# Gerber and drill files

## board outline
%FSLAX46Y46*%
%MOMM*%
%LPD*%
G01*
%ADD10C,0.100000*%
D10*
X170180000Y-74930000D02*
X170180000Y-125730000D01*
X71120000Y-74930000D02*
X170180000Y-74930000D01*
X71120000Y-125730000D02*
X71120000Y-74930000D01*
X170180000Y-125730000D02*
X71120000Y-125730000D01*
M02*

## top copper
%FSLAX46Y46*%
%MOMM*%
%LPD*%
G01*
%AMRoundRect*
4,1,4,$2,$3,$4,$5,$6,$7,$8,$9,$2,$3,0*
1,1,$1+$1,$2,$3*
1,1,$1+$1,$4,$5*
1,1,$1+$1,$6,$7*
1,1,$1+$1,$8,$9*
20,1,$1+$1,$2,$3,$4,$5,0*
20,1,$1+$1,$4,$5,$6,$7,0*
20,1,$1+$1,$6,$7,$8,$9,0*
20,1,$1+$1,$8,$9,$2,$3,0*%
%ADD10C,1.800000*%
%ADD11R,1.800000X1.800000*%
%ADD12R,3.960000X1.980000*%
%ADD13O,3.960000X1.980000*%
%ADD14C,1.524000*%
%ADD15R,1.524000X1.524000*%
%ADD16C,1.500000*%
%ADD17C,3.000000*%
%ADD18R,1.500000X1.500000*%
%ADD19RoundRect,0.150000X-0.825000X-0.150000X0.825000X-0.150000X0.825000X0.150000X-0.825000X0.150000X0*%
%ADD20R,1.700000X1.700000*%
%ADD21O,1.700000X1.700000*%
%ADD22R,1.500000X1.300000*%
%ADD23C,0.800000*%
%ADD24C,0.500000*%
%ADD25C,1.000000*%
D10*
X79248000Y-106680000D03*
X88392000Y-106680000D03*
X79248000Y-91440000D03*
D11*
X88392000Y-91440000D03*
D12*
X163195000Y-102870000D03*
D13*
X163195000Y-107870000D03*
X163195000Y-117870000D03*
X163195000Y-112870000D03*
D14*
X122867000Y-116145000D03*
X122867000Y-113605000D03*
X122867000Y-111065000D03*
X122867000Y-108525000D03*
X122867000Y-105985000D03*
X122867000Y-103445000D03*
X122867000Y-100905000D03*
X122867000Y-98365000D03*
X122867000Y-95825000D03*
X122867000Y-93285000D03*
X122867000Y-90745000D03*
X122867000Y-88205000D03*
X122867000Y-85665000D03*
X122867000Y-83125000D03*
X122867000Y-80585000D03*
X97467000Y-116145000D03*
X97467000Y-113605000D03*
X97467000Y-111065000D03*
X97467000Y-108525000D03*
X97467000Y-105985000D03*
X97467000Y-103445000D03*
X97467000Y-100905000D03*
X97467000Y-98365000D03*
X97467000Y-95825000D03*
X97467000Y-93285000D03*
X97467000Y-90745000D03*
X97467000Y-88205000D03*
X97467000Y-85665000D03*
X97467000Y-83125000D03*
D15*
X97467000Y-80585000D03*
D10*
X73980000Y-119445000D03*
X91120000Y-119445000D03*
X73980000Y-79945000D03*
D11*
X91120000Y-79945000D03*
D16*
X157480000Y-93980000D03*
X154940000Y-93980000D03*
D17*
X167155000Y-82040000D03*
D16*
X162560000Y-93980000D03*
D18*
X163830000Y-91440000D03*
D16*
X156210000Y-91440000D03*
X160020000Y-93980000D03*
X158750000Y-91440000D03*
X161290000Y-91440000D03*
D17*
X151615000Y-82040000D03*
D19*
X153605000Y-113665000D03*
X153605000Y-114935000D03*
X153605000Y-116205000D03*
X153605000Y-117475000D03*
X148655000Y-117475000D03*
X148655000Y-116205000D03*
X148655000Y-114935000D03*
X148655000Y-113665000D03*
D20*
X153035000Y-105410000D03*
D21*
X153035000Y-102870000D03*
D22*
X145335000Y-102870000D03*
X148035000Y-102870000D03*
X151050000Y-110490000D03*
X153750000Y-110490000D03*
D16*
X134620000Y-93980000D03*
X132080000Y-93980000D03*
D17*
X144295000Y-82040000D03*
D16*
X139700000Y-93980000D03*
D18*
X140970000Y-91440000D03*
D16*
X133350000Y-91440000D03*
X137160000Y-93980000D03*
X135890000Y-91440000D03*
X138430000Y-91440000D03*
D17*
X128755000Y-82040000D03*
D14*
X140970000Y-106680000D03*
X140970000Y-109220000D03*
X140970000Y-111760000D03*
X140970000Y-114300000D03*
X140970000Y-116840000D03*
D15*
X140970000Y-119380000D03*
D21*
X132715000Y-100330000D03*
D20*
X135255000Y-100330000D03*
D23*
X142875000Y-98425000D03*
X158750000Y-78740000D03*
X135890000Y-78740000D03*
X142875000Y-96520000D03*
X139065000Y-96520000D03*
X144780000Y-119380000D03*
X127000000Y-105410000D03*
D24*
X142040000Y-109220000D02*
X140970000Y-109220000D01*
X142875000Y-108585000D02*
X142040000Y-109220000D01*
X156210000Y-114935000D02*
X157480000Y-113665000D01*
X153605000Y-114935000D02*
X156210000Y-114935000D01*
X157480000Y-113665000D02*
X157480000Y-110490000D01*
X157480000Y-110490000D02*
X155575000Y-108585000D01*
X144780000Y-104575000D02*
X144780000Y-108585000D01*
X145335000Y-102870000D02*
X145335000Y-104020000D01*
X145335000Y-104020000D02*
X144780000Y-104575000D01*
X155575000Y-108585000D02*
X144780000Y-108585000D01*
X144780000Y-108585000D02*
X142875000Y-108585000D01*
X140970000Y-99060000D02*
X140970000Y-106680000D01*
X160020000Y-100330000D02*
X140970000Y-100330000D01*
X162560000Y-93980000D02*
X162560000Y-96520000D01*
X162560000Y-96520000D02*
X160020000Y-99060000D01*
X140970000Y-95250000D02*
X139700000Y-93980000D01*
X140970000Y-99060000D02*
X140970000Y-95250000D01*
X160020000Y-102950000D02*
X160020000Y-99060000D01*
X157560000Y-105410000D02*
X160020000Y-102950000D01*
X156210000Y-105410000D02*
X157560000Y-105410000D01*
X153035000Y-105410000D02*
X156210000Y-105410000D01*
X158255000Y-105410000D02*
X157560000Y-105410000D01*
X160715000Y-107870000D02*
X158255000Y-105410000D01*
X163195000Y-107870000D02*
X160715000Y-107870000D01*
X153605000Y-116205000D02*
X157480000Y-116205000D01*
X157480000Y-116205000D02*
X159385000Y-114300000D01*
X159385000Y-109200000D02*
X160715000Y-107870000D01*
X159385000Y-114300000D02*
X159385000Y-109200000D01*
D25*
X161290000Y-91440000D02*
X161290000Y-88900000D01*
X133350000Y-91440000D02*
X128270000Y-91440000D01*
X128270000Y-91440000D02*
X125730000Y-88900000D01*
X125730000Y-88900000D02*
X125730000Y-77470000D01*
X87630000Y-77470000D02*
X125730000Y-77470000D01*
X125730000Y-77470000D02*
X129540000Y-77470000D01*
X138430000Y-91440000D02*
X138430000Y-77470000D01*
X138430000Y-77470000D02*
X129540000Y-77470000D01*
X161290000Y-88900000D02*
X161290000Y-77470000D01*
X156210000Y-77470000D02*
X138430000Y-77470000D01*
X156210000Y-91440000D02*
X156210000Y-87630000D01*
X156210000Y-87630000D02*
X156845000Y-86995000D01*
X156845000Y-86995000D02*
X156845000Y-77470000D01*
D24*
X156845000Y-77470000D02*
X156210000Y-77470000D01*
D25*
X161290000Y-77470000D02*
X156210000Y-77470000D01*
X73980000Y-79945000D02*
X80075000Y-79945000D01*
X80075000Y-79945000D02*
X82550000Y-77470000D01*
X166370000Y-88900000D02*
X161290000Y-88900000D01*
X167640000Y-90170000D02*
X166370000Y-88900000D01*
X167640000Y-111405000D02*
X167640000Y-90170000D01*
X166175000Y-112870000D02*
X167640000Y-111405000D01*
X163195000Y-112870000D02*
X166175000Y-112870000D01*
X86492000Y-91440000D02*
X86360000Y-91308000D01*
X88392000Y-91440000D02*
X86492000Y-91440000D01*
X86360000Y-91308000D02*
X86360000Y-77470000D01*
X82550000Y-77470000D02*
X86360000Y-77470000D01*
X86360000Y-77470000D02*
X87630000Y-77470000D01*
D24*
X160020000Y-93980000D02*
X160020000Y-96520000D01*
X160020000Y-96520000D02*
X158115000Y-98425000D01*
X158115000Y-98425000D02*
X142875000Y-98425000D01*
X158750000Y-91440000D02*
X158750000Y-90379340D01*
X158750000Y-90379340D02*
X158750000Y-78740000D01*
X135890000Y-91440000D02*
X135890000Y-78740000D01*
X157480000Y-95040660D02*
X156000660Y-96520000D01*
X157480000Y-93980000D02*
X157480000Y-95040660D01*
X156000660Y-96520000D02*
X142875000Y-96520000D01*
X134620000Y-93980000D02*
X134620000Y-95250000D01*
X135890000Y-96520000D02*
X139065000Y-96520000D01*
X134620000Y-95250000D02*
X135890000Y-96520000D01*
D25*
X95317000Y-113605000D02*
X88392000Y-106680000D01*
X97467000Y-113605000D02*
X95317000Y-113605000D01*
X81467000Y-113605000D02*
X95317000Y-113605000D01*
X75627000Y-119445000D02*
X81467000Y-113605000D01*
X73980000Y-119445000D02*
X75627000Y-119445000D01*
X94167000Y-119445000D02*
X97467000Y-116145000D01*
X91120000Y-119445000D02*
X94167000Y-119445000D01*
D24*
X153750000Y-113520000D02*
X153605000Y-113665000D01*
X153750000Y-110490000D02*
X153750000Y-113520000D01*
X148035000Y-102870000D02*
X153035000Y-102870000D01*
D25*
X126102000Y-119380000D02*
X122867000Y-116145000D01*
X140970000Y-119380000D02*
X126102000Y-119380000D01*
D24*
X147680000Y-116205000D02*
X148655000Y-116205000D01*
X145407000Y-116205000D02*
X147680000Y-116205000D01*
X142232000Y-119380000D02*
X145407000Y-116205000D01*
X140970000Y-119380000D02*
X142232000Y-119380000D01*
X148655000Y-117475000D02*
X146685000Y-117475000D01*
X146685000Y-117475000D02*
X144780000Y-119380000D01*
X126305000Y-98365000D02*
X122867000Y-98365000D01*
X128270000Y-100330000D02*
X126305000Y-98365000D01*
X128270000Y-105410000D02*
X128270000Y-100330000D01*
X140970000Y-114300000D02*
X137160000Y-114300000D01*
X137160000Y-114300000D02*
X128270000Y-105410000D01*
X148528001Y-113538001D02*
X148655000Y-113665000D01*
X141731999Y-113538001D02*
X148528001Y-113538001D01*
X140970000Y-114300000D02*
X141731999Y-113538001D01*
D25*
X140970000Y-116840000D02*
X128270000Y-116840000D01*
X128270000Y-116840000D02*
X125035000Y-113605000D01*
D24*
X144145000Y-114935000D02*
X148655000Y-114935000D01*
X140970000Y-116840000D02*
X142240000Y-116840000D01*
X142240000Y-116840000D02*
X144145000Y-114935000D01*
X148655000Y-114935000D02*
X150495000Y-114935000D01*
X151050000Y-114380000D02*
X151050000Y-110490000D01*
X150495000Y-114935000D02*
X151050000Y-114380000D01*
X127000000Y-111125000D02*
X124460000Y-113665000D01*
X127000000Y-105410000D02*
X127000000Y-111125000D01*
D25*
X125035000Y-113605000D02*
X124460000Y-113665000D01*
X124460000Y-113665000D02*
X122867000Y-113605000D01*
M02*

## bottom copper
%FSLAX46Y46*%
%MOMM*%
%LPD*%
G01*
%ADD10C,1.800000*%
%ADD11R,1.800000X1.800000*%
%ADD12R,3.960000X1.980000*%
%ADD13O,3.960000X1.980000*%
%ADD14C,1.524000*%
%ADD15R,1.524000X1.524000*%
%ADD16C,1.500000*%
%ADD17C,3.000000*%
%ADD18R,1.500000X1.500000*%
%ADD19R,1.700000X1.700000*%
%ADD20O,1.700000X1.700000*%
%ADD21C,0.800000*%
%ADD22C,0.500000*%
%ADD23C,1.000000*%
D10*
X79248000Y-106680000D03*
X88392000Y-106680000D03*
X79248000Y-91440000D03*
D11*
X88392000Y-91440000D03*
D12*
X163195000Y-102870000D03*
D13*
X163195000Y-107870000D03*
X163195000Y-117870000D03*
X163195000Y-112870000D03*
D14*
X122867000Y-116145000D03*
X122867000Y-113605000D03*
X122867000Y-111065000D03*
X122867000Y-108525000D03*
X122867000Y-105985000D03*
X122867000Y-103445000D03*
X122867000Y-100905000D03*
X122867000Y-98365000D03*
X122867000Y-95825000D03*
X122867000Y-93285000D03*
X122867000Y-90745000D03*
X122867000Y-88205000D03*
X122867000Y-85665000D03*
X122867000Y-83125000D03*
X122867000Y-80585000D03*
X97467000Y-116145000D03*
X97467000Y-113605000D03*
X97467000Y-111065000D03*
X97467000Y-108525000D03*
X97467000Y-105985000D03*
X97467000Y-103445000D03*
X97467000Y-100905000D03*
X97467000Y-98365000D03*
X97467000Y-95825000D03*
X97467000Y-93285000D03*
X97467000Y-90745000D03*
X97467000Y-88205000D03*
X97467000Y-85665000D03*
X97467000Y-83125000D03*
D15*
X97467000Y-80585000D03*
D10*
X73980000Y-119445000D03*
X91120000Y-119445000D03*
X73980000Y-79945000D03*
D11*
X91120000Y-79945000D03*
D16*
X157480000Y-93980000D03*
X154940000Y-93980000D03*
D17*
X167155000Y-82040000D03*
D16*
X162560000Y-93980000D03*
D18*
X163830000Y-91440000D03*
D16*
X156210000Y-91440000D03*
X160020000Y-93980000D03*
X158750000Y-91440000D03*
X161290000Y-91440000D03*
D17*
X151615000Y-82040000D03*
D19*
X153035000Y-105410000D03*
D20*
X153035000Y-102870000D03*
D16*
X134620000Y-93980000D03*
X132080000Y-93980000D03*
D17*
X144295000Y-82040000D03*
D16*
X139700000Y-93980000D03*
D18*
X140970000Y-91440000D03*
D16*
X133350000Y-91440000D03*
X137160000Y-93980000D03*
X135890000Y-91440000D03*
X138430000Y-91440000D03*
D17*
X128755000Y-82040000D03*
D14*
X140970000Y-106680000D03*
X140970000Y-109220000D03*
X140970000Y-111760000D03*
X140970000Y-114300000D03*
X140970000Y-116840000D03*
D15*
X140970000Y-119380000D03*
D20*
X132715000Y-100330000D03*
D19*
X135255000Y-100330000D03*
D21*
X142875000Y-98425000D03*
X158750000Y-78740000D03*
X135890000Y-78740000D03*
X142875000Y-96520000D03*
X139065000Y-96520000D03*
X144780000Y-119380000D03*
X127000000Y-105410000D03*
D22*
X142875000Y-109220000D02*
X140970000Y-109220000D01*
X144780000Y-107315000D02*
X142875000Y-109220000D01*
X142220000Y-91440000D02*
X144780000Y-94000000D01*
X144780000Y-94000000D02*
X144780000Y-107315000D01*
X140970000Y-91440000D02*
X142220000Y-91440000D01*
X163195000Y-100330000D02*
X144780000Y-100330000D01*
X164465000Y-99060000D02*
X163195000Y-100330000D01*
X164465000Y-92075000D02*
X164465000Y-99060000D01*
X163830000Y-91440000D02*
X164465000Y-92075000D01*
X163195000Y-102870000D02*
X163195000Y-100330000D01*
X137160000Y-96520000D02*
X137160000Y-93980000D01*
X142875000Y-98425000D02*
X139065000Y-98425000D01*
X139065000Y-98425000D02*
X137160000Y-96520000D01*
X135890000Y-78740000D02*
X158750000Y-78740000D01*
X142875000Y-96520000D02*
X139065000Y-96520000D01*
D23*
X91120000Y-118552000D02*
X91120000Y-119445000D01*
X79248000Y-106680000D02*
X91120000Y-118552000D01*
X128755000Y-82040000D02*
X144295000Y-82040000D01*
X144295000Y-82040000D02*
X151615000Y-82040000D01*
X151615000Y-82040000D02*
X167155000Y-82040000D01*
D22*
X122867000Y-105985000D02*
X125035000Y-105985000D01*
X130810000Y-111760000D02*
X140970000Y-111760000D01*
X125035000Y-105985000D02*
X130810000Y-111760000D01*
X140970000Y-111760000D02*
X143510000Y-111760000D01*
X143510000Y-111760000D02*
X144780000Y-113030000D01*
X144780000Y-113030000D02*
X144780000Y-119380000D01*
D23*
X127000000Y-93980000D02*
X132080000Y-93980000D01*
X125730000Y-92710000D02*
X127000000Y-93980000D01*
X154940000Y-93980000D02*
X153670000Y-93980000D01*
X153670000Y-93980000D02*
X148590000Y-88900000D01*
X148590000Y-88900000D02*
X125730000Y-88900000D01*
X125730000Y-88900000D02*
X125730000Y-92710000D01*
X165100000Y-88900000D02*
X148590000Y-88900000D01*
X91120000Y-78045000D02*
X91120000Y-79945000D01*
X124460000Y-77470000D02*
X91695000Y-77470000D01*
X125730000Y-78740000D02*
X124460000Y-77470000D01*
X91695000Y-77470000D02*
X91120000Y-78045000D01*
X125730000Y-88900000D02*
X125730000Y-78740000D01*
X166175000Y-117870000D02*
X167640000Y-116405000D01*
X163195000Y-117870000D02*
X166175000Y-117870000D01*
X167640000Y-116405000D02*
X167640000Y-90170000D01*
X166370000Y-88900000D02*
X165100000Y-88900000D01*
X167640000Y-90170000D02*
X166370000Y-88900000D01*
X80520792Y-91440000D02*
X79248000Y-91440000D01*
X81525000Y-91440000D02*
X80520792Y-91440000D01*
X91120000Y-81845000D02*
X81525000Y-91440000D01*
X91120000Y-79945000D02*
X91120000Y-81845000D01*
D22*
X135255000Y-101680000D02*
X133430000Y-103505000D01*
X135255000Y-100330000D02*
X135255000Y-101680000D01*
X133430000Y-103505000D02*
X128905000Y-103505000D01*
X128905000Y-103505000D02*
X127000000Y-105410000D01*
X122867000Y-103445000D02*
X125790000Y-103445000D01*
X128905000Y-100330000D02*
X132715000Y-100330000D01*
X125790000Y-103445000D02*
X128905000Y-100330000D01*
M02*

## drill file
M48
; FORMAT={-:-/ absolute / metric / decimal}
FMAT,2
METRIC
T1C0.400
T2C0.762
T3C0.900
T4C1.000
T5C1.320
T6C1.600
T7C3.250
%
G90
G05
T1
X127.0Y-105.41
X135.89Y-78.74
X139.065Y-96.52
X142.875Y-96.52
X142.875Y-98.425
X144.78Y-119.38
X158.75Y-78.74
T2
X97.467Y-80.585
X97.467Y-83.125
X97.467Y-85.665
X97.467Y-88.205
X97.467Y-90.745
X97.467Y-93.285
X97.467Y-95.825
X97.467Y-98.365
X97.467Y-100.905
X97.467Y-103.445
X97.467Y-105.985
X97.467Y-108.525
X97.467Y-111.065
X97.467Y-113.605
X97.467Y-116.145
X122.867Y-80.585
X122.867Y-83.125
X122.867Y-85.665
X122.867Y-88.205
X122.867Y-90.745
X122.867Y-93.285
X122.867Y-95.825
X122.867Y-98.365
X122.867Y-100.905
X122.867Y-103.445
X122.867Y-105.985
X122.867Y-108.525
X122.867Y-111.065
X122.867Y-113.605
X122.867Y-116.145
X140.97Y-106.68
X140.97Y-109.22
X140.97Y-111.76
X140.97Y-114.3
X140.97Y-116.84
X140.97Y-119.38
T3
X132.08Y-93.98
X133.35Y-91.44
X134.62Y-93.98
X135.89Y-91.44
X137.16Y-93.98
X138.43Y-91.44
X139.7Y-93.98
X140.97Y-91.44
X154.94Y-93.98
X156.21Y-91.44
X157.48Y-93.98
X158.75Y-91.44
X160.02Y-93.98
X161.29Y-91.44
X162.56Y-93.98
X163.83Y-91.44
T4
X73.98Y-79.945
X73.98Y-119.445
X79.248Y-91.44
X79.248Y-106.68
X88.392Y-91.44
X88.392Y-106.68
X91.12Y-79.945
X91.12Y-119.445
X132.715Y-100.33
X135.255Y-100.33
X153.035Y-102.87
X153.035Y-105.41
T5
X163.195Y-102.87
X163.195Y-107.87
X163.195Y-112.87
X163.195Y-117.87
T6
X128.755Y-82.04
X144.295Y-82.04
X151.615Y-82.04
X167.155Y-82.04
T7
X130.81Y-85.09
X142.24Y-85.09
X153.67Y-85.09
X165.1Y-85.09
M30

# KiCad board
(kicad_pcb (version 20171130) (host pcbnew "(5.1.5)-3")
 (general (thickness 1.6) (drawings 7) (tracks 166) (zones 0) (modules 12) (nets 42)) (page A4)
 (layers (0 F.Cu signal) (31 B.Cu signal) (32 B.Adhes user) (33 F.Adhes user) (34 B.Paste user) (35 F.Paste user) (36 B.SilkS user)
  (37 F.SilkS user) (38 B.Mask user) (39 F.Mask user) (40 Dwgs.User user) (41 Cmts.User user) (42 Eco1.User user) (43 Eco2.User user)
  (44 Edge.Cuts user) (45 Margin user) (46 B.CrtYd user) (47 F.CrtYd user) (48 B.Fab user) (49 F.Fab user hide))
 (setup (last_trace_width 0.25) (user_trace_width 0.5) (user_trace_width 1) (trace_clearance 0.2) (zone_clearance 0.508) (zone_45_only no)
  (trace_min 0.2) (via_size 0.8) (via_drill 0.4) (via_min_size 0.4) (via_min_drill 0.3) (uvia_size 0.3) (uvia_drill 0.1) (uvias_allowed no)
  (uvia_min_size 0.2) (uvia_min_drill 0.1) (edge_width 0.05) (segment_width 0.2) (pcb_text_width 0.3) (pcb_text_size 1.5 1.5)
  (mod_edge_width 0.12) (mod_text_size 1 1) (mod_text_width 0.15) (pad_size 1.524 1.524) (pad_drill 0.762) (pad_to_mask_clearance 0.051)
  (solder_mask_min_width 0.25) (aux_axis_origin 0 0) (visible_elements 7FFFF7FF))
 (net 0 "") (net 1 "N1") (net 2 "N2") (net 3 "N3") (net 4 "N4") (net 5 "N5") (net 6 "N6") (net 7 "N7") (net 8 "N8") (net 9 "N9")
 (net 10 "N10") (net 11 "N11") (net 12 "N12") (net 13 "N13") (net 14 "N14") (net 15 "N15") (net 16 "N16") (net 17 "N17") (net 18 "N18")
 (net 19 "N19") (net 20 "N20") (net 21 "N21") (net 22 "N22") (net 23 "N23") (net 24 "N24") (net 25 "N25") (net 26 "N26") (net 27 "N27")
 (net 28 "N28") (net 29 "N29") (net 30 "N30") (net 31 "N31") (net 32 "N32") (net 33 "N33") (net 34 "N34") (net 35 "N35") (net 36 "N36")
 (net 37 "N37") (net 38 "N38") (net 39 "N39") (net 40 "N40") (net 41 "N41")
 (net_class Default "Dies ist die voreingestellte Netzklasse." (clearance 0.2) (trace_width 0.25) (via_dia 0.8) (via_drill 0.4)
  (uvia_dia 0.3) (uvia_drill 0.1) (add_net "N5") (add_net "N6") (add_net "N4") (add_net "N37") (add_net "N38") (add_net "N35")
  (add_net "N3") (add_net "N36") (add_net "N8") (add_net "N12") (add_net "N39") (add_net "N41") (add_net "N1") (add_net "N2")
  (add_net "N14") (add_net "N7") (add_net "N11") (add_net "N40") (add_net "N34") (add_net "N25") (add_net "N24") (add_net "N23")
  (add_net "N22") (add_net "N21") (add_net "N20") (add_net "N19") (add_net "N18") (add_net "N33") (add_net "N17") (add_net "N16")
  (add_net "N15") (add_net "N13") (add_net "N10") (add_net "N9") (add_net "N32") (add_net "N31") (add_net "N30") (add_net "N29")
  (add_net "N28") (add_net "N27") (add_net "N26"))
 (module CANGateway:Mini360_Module (layer F.Cu) (at 83.82 99.06 270)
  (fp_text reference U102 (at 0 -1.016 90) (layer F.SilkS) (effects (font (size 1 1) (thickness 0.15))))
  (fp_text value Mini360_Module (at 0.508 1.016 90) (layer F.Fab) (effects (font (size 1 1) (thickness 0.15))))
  (pad 4 thru_hole circle (at 7.62 4.572 270) (size 1.8 1.8) (drill 1) (layers *.Cu *.Mask) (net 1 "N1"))
  (pad 3 thru_hole circle (at 7.62 -4.572 270) (size 1.8 1.8) (drill 1) (layers *.Cu *.Mask) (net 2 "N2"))
  (pad 2 thru_hole circle (at -7.62 4.572 270) (size 1.8 1.8) (drill 1) (layers *.Cu *.Mask) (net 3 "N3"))
  (pad 1 thru_hole rect (at -7.62 -4.572 270) (size 1.8 1.8) (drill 1) (layers *.Cu *.Mask) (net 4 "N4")))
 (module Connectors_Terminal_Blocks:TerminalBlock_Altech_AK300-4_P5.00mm (layer F.Cu) (at 163.195 102.87 270)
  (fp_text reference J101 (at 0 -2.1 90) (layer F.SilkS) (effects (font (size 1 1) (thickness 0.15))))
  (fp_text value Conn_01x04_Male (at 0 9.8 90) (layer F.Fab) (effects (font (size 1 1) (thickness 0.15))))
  (pad 1 thru_hole rect (at 0 0 270) (size 1.98 3.96) (drill 1.32) (layers *.Cu *.Mask) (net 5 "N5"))
  (pad 2 thru_hole oval (at 5 0 270) (size 1.98 3.96) (drill 1.32) (layers *.Cu *.Mask) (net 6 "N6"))
  (pad 4 thru_hole oval (at 15 0 270) (size 1.98 3.96) (drill 1.32) (layers *.Cu *.Mask) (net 3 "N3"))
  (pad 3 thru_hole oval (at 10 0 270) (size 1.98 3.96) (drill 1.32) (layers *.Cu *.Mask) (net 4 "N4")))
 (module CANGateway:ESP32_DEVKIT (layer F.Cu) (at 110.167 95.825)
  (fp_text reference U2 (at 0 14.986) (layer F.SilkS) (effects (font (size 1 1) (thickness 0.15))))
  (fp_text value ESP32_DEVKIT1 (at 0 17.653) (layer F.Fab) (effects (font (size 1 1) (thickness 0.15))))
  (pad 30 thru_hole circle (at 12.7 20.32) (size 1.524 1.524) (drill 0.762) (layers *.Cu *.Mask) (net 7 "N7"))
  (pad 29 thru_hole circle (at 12.7 17.78) (size 1.524 1.524) (drill 0.762) (layers *.Cu *.Mask) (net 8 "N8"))
  (pad 28 thru_hole circle (at 12.7 15.24) (size 1.524 1.524) (drill 0.762) (layers *.Cu *.Mask) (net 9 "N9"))
  (pad 27 thru_hole circle (at 12.7 12.7) (size 1.524 1.524) (drill 0.762) (layers *.Cu *.Mask) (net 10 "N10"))
  (pad 26 thru_hole circle (at 12.7 10.16) (size 1.524 1.524) (drill 0.762) (layers *.Cu *.Mask) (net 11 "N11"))
  (pad 25 thru_hole circle (at 12.7 7.62) (size 1.524 1.524) (drill 0.762) (layers *.Cu *.Mask) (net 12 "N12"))
  (pad 24 thru_hole circle (at 12.7 5.08) (size 1.524 1.524) (drill 0.762) (layers *.Cu *.Mask) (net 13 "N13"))
  (pad 23 thru_hole circle (at 12.7 2.54) (size 1.524 1.524) (drill 0.762) (layers *.Cu *.Mask) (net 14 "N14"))
  (pad 22 thru_hole circle (at 12.7 0) (size 1.524 1.524) (drill 0.762) (layers *.Cu *.Mask) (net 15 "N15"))
  (pad 21 thru_hole circle (at 12.7 -2.54) (size 1.524 1.524) (drill 0.762) (layers *.Cu *.Mask) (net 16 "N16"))
  (pad 20 thru_hole circle (at 12.7 -5.08) (size 1.524 1.524) (drill 0.762) (layers *.Cu *.Mask) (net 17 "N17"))
  (pad 19 thru_hole circle (at 12.7 -7.62) (size 1.524 1.524) (drill 0.762) (layers *.Cu *.Mask) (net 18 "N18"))
  (pad 18 thru_hole circle (at 12.7 -10.16) (size 1.524 1.524) (drill 0.762) (layers *.Cu *.Mask) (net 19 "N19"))
  (pad 17 thru_hole circle (at 12.7 -12.7) (size 1.524 1.524) (drill 0.762) (layers *.Cu *.Mask) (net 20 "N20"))
  (pad 16 thru_hole circle (at 12.7 -15.24) (size 1.524 1.524) (drill 0.762) (layers *.Cu *.Mask) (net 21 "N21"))
  (pad 15 thru_hole circle (at -12.7 20.32) (size 1.524 1.524) (drill 0.762) (layers *.Cu *.Mask) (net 1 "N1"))
  (pad 14 thru_hole circle (at -12.7 17.78) (size 1.524 1.524) (drill 0.762) (layers *.Cu *.Mask) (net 2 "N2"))
  (pad 13 thru_hole circle (at -12.7 15.24) (size 1.524 1.524) (drill 0.762) (layers *.Cu *.Mask) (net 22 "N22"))
  (pad 12 thru_hole circle (at -12.7 12.7) (size 1.524 1.524) (drill 0.762) (layers *.Cu *.Mask) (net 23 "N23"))
  (pad 11 thru_hole circle (at -12.7 10.16) (size 1.524 1.524) (drill 0.762) (layers *.Cu *.Mask) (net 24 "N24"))
  (pad 10 thru_hole circle (at -12.7 7.62) (size 1.524 1.524) (drill 0.762) (layers *.Cu *.Mask) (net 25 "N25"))
  (pad 9 thru_hole circle (at -12.7 5.08) (size 1.524 1.524) (drill 0.762) (layers *.Cu *.Mask) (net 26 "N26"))
  (pad 8 thru_hole circle (at -12.7 2.54) (size 1.524 1.524) (drill 0.762) (layers *.Cu *.Mask) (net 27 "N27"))
  (pad 7 thru_hole circle (at -12.7 0) (size 1.524 1.524) (drill 0.762) (layers *.Cu *.Mask) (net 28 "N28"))
  (pad 6 thru_hole circle (at -12.7 -2.54) (size 1.524 1.524) (drill 0.762) (layers *.Cu *.Mask) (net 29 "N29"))
  (pad 5 thru_hole circle (at -12.7 -5.08) (size 1.524 1.524) (drill 0.762) (layers *.Cu *.Mask) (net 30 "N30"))
  (pad 4 thru_hole circle (at -12.7 -7.62) (size 1.524 1.524) (drill 0.762) (layers *.Cu *.Mask) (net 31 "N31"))
  (pad 3 thru_hole circle (at -12.7 -10.16) (size 1.524 1.524) (drill 0.762) (layers *.Cu *.Mask) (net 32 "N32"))
  (pad 2 thru_hole circle (at -12.7 -12.7) (size 1.524 1.524) (drill 0.762) (layers *.Cu *.Mask) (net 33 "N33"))
  (pad 1 thru_hole rect (at -12.7 -15.24) (size 1.524 1.524) (drill 0.762) (layers *.Cu *.Mask) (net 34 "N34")))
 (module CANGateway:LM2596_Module (layer F.Cu) (at 82.55 99.695 270)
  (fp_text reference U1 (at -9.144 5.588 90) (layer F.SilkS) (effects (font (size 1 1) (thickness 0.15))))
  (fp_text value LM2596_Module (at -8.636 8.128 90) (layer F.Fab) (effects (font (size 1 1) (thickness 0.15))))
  (pad 4 thru_hole circle (at 19.75 8.57 270) (size 1.8 1.8) (drill 1) (layers *.Cu *.Mask) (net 2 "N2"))
  (pad 3 thru_hole circle (at 19.75 -8.57 270) (size 1.8 1.8) (drill 1) (layers *.Cu *.Mask) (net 1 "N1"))
  (pad 2 thru_hole circle (at -19.75 8.57 270) (size 1.8 1.8) (drill 1) (layers *.Cu *.Mask) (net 4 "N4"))
  (pad 1 thru_hole rect (at -19.75 -8.57 270) (size 1.8 1.8) (drill 1) (layers *.Cu *.Mask) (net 3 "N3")))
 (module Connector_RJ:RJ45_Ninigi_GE (layer F.Cu) (at 163.83 91.44 180)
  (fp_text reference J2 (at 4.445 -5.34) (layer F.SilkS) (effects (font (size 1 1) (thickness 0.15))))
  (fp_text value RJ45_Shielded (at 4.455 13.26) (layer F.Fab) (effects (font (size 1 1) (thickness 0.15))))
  (pad 6 thru_hole circle (at 6.35 -2.54) (size 1.5 1.5) (drill 0.9) (layers *.Cu *.Mask) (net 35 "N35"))
  (pad 8 thru_hole circle (at 8.89 -2.54) (size 1.5 1.5) (drill 0.9) (layers *.Cu *.Mask) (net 3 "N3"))
  (pad SH thru_hole circle (at -3.325 9.4 180) (size 3 3) (drill 1.6) (layers *.Cu *.Mask) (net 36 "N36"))
  (pad 2 thru_hole circle (at 1.27 -2.54) (size 1.5 1.5) (drill 0.9) (layers *.Cu *.Mask) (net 6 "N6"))
  (pad 1 thru_hole rect (at 0 0) (size 1.5 1.5) (drill 0.9) (layers *.Cu *.Mask) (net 5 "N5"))
  (pad 7 thru_hole circle (at 7.62 0) (size 1.5 1.5) (drill 0.9) (layers *.Cu *.Mask) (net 4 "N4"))
  (pad 4 thru_hole circle (at 3.81 -2.54) (size 1.5 1.5) (drill 0.9) (layers *.Cu *.Mask) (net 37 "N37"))
  (pad 5 thru_hole circle (at 5.08 0) (size 1.5 1.5) (drill 0.9) (layers *.Cu *.Mask) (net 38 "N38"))
  (pad 3 thru_hole circle (at 2.54 0) (size 1.5 1.5) (drill 0.9) (layers *.Cu *.Mask) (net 4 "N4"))
  (pad "" np_thru_hole circle (at -1.27 6.35 180) (size 3.25 3.25) (drill 3.25) (layers *.Cu *.Mask))
  (pad SH thru_hole circle (at 12.215 9.4) (size 3 3) (drill 1.6) (layers *.Cu *.Mask) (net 36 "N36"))
  (pad "" np_thru_hole circle (at 10.16 6.35) (size 3.25 3.25) (drill 3.25) (layers *.Cu *.Mask)))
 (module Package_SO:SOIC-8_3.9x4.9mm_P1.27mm (layer F.Cu) (at 151.13 115.57)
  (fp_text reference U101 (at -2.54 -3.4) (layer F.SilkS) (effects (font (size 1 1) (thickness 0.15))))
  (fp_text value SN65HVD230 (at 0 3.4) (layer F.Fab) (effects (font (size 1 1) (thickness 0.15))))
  (pad 8 smd roundrect (at 2.475 -1.905) (size 1.95 0.6) (layers F.Cu F.Paste F.Mask) (roundrect_rratio 0.25) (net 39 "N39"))
  (pad 7 smd roundrect (at 2.475 -0.635) (size 1.95 0.6) (layers F.Cu F.Paste F.Mask) (roundrect_rratio 0.25) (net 5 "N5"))
  (pad 6 smd roundrect (at 2.475 0.635) (size 1.95 0.6) (layers F.Cu F.Paste F.Mask) (roundrect_rratio 0.25) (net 6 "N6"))
  (pad 5 smd roundrect (at 2.475 1.905) (size 1.95 0.6) (layers F.Cu F.Paste F.Mask) (roundrect_rratio 0.25) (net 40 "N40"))
  (pad 4 smd roundrect (at -2.475 1.905) (size 1.95 0.6) (layers F.Cu F.Paste F.Mask) (roundrect_rratio 0.25) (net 11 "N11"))
  (pad 3 smd roundrect (at -2.475 0.635) (size 1.95 0.6) (layers F.Cu F.Paste F.Mask) (roundrect_rratio 0.25) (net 7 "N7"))
  (pad 2 smd roundrect (at -2.475 -0.635) (size 1.95 0.6) (layers F.Cu F.Paste F.Mask) (roundrect_rratio 0.25) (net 8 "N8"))
  (pad 1 smd roundrect (at -2.475 -1.905) (size 1.95 0.6) (layers F.Cu F.Paste F.Mask) (roundrect_rratio 0.25) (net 14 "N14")))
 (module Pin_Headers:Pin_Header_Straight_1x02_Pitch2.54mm (layer F.Cu) (at 153.035 105.41 180)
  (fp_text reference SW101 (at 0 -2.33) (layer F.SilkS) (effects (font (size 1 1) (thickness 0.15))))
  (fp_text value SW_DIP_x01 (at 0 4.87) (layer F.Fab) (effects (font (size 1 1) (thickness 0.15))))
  (pad 1 thru_hole rect (at 0 0 180) (size 1.7 1.7) (drill 1) (layers *.Cu *.Mask) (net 6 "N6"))
  (pad 2 thru_hole oval (at 0 2.54 180) (size 1.7 1.7) (drill 1) (layers *.Cu *.Mask) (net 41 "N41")))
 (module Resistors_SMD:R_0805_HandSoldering (layer F.Cu) (at 146.685 102.87)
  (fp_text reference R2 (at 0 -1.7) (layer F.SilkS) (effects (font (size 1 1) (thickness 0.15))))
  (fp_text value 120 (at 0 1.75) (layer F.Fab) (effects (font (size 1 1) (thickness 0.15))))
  (pad 1 smd rect (at -1.35 0) (size 1.5 1.3) (layers F.Cu F.Paste F.Mask) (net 5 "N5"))
  (pad 2 smd rect (at 1.35 0) (size 1.5 1.3) (layers F.Cu F.Paste F.Mask) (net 41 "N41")))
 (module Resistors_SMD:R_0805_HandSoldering (layer F.Cu) (at 152.4 110.49)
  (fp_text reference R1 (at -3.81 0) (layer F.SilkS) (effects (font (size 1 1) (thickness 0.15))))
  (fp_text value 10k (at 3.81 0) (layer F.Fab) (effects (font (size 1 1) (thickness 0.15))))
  (pad 1 smd rect (at -1.35 0) (size 1.5 1.3) (layers F.Cu F.Paste F.Mask) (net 8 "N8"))
  (pad 2 smd rect (at 1.35 0) (size 1.5 1.3) (layers F.Cu F.Paste F.Mask) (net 39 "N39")))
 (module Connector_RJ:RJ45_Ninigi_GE (layer F.Cu) (at 140.97 91.44 180)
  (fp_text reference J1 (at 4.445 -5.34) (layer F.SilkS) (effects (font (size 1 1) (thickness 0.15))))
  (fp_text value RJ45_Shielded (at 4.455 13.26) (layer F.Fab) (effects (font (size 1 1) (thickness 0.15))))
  (pad 6 thru_hole circle (at 6.35 -2.54) (size 1.5 1.5) (drill 0.9) (layers *.Cu *.Mask) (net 35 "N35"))
  (pad 8 thru_hole circle (at 8.89 -2.54) (size 1.5 1.5) (drill 0.9) (layers *.Cu *.Mask) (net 3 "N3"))
  (pad SH thru_hole circle (at -3.325 9.4 180) (size 3 3) (drill 1.6) (layers *.Cu *.Mask) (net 36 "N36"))
  (pad 2 thru_hole circle (at 1.27 -2.54) (size 1.5 1.5) (drill 0.9) (layers *.Cu *.Mask) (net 6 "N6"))
  (pad 1 thru_hole rect (at 0 0) (size 1.5 1.5) (drill 0.9) (layers *.Cu *.Mask) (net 5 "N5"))
  (pad 7 thru_hole circle (at 7.62 0) (size 1.5 1.5) (drill 0.9) (layers *.Cu *.Mask) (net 4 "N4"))
  (pad 4 thru_hole circle (at 3.81 -2.54) (size 1.5 1.5) (drill 0.9) (layers *.Cu *.Mask) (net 37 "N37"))
  (pad 5 thru_hole circle (at 5.08 0) (size 1.5 1.5) (drill 0.9) (layers *.Cu *.Mask) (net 38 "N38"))
  (pad 3 thru_hole circle (at 2.54 0) (size 1.5 1.5) (drill 0.9) (layers *.Cu *.Mask) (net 4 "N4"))
  (pad "" np_thru_hole circle (at -1.27 6.35 180) (size 3.25 3.25) (drill 3.25) (layers *.Cu *.Mask))
  (pad SH thru_hole circle (at 12.215 9.4) (size 3 3) (drill 1.6) (layers *.Cu *.Mask) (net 36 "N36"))
  (pad "" np_thru_hole circle (at 10.16 6.35) (size 3.25 3.25) (drill 3.25) (layers *.Cu *.Mask)))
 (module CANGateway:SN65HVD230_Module (layer F.Cu) (at 140.97 121.92 180)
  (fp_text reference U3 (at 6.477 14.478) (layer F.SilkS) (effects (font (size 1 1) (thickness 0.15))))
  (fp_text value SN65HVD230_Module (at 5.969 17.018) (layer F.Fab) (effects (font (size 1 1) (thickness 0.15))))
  (pad 6 thru_hole circle (at 0 15.24 180) (size 1.524 1.524) (drill 0.762) (layers *.Cu *.Mask) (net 6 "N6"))
  (pad 5 thru_hole circle (at 0 12.7 180) (size 1.524 1.524) (drill 0.762) (layers *.Cu *.Mask) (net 5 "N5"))
  (pad 4 thru_hole circle (at 0 10.16 180) (size 1.524 1.524) (drill 0.762) (layers *.Cu *.Mask) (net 11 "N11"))
  (pad 3 thru_hole circle (at 0 7.62 180) (size 1.524 1.524) (drill 0.762) (layers *.Cu *.Mask) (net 14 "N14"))
  (pad 2 thru_hole circle (at 0 5.08 180) (size 1.524 1.524) (drill 0.762) (layers *.Cu *.Mask) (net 8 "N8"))
  (pad 1 thru_hole rect (at 0 2.54 180) (size 1.524 1.524) (drill 0.762) (layers *.Cu *.Mask) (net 7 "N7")))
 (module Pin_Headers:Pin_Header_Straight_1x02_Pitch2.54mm (layer F.Cu) (at 135.255 100.33 270)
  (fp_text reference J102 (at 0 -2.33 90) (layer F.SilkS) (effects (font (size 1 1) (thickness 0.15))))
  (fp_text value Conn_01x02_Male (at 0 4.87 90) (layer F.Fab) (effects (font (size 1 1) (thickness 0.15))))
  (pad 2 thru_hole oval (at 0 2.54 270) (size 1.7 1.7) (drill 1) (layers *.Cu *.Mask) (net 12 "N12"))
  (pad 1 thru_hole rect (at 0 0 270) (size 1.7 1.7) (drill 1) (layers *.Cu *.Mask) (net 8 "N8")))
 (gr_line (start 170.18 74.93) (end 170.18 125.73) (layer Edge.Cuts) (width 0.1))
 (gr_line (start 71.12 74.93) (end 170.18 74.93) (layer Edge.Cuts) (width 0.1))
 (gr_line (start 71.12 125.73) (end 71.12 74.93) (layer Edge.Cuts) (width 0.1))
 (gr_line (start 170.18 125.73) (end 71.12 125.73) (layer Edge.Cuts) (width 0.1))
 (segment (start 142.04 109.22) (end 140.97 109.22) (width 0.5) (layer F.Cu) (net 5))
 (segment (start 142.875 108.585) (end 142.04 109.22) (width 0.5) (layer F.Cu) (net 5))
 (segment (start 142.875 109.22) (end 140.97 109.22) (width 0.5) (layer B.Cu) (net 5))
 (segment (start 144.78 107.315) (end 142.875 109.22) (width 0.5) (layer B.Cu) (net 5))
 (segment (start 142.22 91.44) (end 144.78 94) (width 0.5) (layer B.Cu) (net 5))
 (segment (start 144.78 94) (end 144.78 107.315) (width 0.5) (layer B.Cu) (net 5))
 (segment (start 140.97 91.44) (end 142.22 91.44) (width 0.5) (layer B.Cu) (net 5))
 (segment (start 156.21 114.935) (end 157.48 113.665) (width 0.5) (layer F.Cu) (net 5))
 (segment (start 153.605 114.935) (end 156.21 114.935) (width 0.5) (layer F.Cu) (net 5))
 (segment (start 157.48 113.665) (end 157.48 110.49) (width 0.5) (layer F.Cu) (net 5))
 (segment (start 157.48 110.49) (end 155.575 108.585) (width 0.5) (layer F.Cu) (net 5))
 (segment (start 163.195 100.33) (end 144.78 100.33) (width 0.5) (layer B.Cu) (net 5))
 (segment (start 164.465 99.06) (end 163.195 100.33) (width 0.5) (layer B.Cu) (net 5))
 (segment (start 164.465 92.075) (end 164.465 99.06) (width 0.5) (layer B.Cu) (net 5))
 (segment (start 163.83 91.44) (end 164.465 92.075) (width 0.5) (layer B.Cu) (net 5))
 (segment (start 144.78 104.575) (end 144.78 108.585) (width 0.5) (layer F.Cu) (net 5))
 (segment (start 145.335 102.87) (end 145.335 104.02) (width 0.5) (layer F.Cu) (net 5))
 (segment (start 145.335 104.02) (end 144.78 104.575) (width 0.5) (layer F.Cu) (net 5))
 (segment (start 155.575 108.585) (end 144.78 108.585) (width 0.5) (layer F.Cu) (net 5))
 (segment (start 144.78 108.585) (end 142.875 108.585) (width 0.5) (layer F.Cu) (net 5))
 (segment (start 163.195 102.87) (end 163.195 100.33) (width 0.5) (layer B.Cu) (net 5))
 (segment (start 140.97 99.06) (end 140.97 106.68) (width 0.5) (layer F.Cu) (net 6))
 (segment (start 160.02 100.33) (end 140.97 100.33) (width 0.5) (layer F.Cu) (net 6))
 (segment (start 162.56 93.98) (end 162.56 96.52) (width 0.5) (layer F.Cu) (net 6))
 (segment (start 162.56 96.52) (end 160.02 99.06) (width 0.5) (layer F.Cu) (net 6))
 (segment (start 140.97 95.25) (end 139.7 93.98) (width 0.5) (layer F.Cu) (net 6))
 (segment (start 140.97 99.06) (end 140.97 95.25) (width 0.5) (layer F.Cu) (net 6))
 (segment (start 160.02 102.95) (end 160.02 99.06) (width 0.5) (layer F.Cu) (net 6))
 (segment (start 157.56 105.41) (end 160.02 102.95) (width 0.5) (layer F.Cu) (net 6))
 (segment (start 156.21 105.41) (end 157.56 105.41) (width 0.5) (layer F.Cu) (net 6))
 (segment (start 153.035 105.41) (end 156.21 105.41) (width 0.5) (layer F.Cu) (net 6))
 (segment (start 158.255 105.41) (end 157.56 105.41) (width 0.5) (layer F.Cu) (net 6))
 (segment (start 160.715 107.87) (end 158.255 105.41) (width 0.5) (layer F.Cu) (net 6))
 (segment (start 163.195 107.87) (end 160.715 107.87) (width 0.5) (layer F.Cu) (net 6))
 (segment (start 153.605 116.205) (end 157.48 116.205) (width 0.5) (layer F.Cu) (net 6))
 (segment (start 157.48 116.205) (end 159.385 114.3) (width 0.5) (layer F.Cu) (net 6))
 (segment (start 159.385 109.2) (end 160.715 107.87) (width 0.5) (layer F.Cu) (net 6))
 (segment (start 159.385 114.3) (end 159.385 109.2) (width 0.5) (layer F.Cu) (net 6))
 (segment (start 161.29 91.44) (end 161.29 88.9) (width 1) (layer F.Cu) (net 4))
 (segment (start 133.35 91.44) (end 128.27 91.44) (width 1) (layer F.Cu) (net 4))
 (segment (start 128.27 91.44) (end 125.73 88.9) (width 1) (layer F.Cu) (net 4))
 (segment (start 125.73 88.9) (end 125.73 77.47) (width 1) (layer F.Cu) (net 4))
 (segment (start 87.63 77.47) (end 125.73 77.47) (width 1) (layer F.Cu) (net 4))
 (segment (start 125.73 77.47) (end 129.54 77.47) (width 1) (layer F.Cu) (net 4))
 (segment (start 138.43 91.44) (end 138.43 77.47) (width 1) (layer F.Cu) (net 4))
 (segment (start 138.43 77.47) (end 129.54 77.47) (width 1) (layer F.Cu) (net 4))
 (segment (start 161.29 88.9) (end 161.29 77.47) (width 1) (layer F.Cu) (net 4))
 (segment (start 156.21 77.47) (end 138.43 77.47) (width 1) (layer F.Cu) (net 4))
 (segment (start 156.21 91.44) (end 156.21 87.63) (width 1) (layer F.Cu) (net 4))
 (segment (start 156.21 87.63) (end 156.845 86.995) (width 1) (layer F.Cu) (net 4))
 (segment (start 156.845 86.995) (end 156.845 77.47) (width 1) (layer F.Cu) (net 4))
 (segment (start 156.845 77.47) (end 156.21 77.47) (width 0.5) (layer F.Cu) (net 4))
 (segment (start 161.29 77.47) (end 156.21 77.47) (width 1) (layer F.Cu) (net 4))
 (segment (start 73.98 79.945) (end 80.075 79.945) (width 1) (layer F.Cu) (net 4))
 (segment (start 80.075 79.945) (end 82.55 77.47) (width 1) (layer F.Cu) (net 4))
 (segment (start 166.37 88.9) (end 161.29 88.9) (width 1) (layer F.Cu) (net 4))
 (segment (start 167.64 90.17) (end 166.37 88.9) (width 1) (layer F.Cu) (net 4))
 (segment (start 167.64 111.405) (end 167.64 90.17) (width 1) (layer F.Cu) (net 4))
 (segment (start 166.175 112.87) (end 167.64 111.405) (width 1) (layer F.Cu) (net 4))
 (segment (start 163.195 112.87) (end 166.175 112.87) (width 1) (layer F.Cu) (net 4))
 (segment (start 86.492 91.44) (end 86.36 91.308) (width 1) (layer F.Cu) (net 4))
 (segment (start 88.392 91.44) (end 86.492 91.44) (width 1) (layer F.Cu) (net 4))
 (segment (start 86.36 91.308) (end 86.36 77.47) (width 1) (layer F.Cu) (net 4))
 (segment (start 82.55 77.47) (end 86.36 77.47) (width 1) (layer F.Cu) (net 4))
 (segment (start 86.36 77.47) (end 87.63 77.47) (width 1) (layer F.Cu) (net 4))
 (segment (start 160.02 93.98) (end 160.02 96.52) (width 0.5) (layer F.Cu) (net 37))
 (segment (start 160.02 96.52) (end 158.115 98.425) (width 0.5) (layer F.Cu) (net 37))
 (via (at 142.875 98.425) (size 0.8) (drill 0.4) (layers F.Cu B.Cu) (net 37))
 (segment (start 158.115 98.425) (end 142.875 98.425) (width 0.5) (layer F.Cu) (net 37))
 (segment (start 137.16 96.52) (end 137.16 93.98) (width 0.5) (layer B.Cu) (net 37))
 (segment (start 142.875 98.425) (end 139.065 98.425) (width 0.5) (layer B.Cu) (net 37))
 (segment (start 139.065 98.425) (end 137.16 96.52) (width 0.5) (layer B.Cu) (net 37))
 (segment (start 158.75 91.44) (end 158.75 90.37934) (width 0.5) (layer F.Cu) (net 38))
 (via (at 158.75 78.74) (size 0.8) (drill 0.4) (layers F.Cu B.Cu) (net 38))
 (segment (start 158.75 90.37934) (end 158.75 78.74) (width 0.5) (layer F.Cu) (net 38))
 (segment (start 135.89 91.44) (end 135.89 78.74) (width 0.5) (layer F.Cu) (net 38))
 (via (at 135.89 78.74) (size 0.8) (drill 0.4) (layers F.Cu B.Cu) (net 38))
 (segment (start 135.89 78.74) (end 158.75 78.74) (width 0.5) (layer B.Cu) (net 38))
 (segment (start 157.48 95.04066) (end 156.00066 96.52) (width 0.5) (layer F.Cu) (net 35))
 (segment (start 157.48 93.98) (end 157.48 95.04066) (width 0.5) (layer F.Cu) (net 35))
 (via (at 142.875 96.52) (size 0.8) (drill 0.4) (layers F.Cu B.Cu) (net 35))
 (segment (start 156.00066 96.52) (end 142.875 96.52) (width 0.5) (layer F.Cu) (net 35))
 (segment (start 142.875 96.52) (end 139.065 96.52) (width 0.5) (layer B.Cu) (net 35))
 (via (at 139.065 96.52) (size 0.8) (drill 0.4) (layers F.Cu B.Cu) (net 35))
 (segment (start 134.62 93.98) (end 134.62 95.25) (width 0.5) (layer F.Cu) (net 35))
 (segment (start 135.89 96.52) (end 139.065 96.52) (width 0.5) (layer F.Cu) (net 35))
 (segment (start 134.62 95.25) (end 135.89 96.52) (width 0.5) (layer F.Cu) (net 35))
 (segment (start 95.317 113.605) (end 88.392 106.68) (width 1) (layer F.Cu) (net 2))
 (segment (start 97.467 113.605) (end 95.317 113.605) (width 1) (layer F.Cu) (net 2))
 (segment (start 81.467 113.605) (end 95.317 113.605) (width 1) (layer F.Cu) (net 2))
 (segment (start 75.627 119.445) (end 81.467 113.605) (width 1) (layer F.Cu) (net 2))
 (segment (start 73.98 119.445) (end 75.627 119.445) (width 1) (layer F.Cu) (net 2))
 (segment (start 94.167 119.445) (end 97.467 116.145) (width 1) (layer F.Cu) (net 1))
 (segment (start 91.12 119.445) (end 94.167 119.445) (width 1) (layer F.Cu) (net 1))
 (segment (start 91.12 118.552) (end 91.12 119.445) (width 1) (layer B.Cu) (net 1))
 (segment (start 79.248 106.68) (end 91.12 118.552) (width 1) (layer B.Cu) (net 1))
 (segment (start 128.755 82.04) (end 144.295 82.04) (width 1) (layer B.Cu) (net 36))
 (segment (start 144.295 82.04) (end 151.615 82.04) (width 1) (layer B.Cu) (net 36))
 (segment (start 151.615 82.04) (end 167.155 82.04) (width 1) (layer B.Cu) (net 36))
 (segment (start 153.75 113.52) (end 153.605 113.665) (width 0.5) (layer F.Cu) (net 39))
 (segment (start 153.75 110.49) (end 153.75 113.52) (width 0.5) (layer F.Cu) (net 39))
 (segment (start 148.035 102.87) (end 153.035 102.87) (width 0.5) (layer F.Cu) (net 41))
 (segment (start 126.102 119.38) (end 122.867 116.145) (width 1) (layer F.Cu) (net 7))
 (segment (start 140.97 119.38) (end 126.102 119.38) (width 1) (layer F.Cu) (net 7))
 (segment (start 147.68 116.205) (end 148.655 116.205) (width 0.5) (layer F.Cu) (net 7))
 (segment (start 145.407 116.205) (end 147.68 116.205) (width 0.5) (layer F.Cu) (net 7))
 (segment (start 142.232 119.38) (end 145.407 116.205) (width 0.5) (layer F.Cu) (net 7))
 (segment (start 140.97 119.38) (end 142.232 119.38) (width 0.5) (layer F.Cu) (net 7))
 (segment (start 122.867 105.985) (end 125.035 105.985) (width 0.5) (layer B.Cu) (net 11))
 (segment (start 130.81 111.76) (end 140.97 111.76) (width 0.5) (layer B.Cu) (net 11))
 (segment (start 125.035 105.985) (end 130.81 111.76) (width 0.5) (layer B.Cu) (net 11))
 (segment (start 140.97 111.76) (end 143.51 111.76) (width 0.5) (layer B.Cu) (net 11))
 (segment (start 143.51 111.76) (end 144.78 113.03) (width 0.5) (layer B.Cu) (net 11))
 (segment (start 148.655 117.475) (end 146.685 117.475) (width 0.5) (layer F.Cu) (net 11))
 (segment (start 146.685 117.475) (end 144.78 119.38) (width 0.5) (layer F.Cu) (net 11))
 (via (at 144.78 119.38) (size 0.8) (drill 0.4) (layers F.Cu B.Cu) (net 11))
 (segment (start 144.78 113.03) (end 144.78 119.38) (width 0.5) (layer B.Cu) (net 11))
 (segment (start 126.305 98.365) (end 122.867 98.365) (width 0.5) (layer F.Cu) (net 14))
 (segment (start 128.27 100.33) (end 126.305 98.365) (width 0.5) (layer F.Cu) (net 14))
 (segment (start 128.27 105.41) (end 128.27 100.33) (width 0.5) (layer F.Cu) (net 14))
 (segment (start 140.97 114.3) (end 137.16 114.3) (width 0.5) (layer F.Cu) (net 14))
 (segment (start 137.16 114.3) (end 128.27 105.41) (width 0.5) (layer F.Cu) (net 14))
 (segment (start 148.528001 113.538001) (end 148.655 113.665) (width 0.5) (layer F.Cu) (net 14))
 (segment (start 141.731999 113.538001) (end 148.528001 113.538001) (width 0.5) (layer F.Cu) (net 14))
 (segment (start 140.97 114.3) (end 141.731999 113.538001) (width 0.5) (layer F.Cu) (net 14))
 (segment (start 127 93.98) (end 132.08 93.98) (width 1) (layer B.Cu) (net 3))
 (segment (start 125.73 92.71) (end 127 93.98) (width 1) (layer B.Cu) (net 3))
 (segment (start 154.94 93.98) (end 153.67 93.98) (width 1) (layer B.Cu) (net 3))
 (segment (start 153.67 93.98) (end 148.59 88.9) (width 1) (layer B.Cu) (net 3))
 (segment (start 148.59 88.9) (end 125.73 88.9) (width 1) (layer B.Cu) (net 3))
 (segment (start 125.73 88.9) (end 125.73 92.71) (width 1) (layer B.Cu) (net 3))
 (segment (start 165.1 88.9) (end 148.59 88.9) (width 1) (layer B.Cu) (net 3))
 (segment (start 91.12 78.045) (end 91.12 79.945) (width 1) (layer B.Cu) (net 3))
 (segment (start 124.46 77.47) (end 91.695 77.47) (width 1) (layer B.Cu) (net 3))
 (segment (start 125.73 78.74) (end 124.46 77.47) (width 1) (layer B.Cu) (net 3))
 (segment (start 91.695 77.47) (end 91.12 78.045) (width 1) (layer B.Cu) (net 3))
 (segment (start 125.73 88.9) (end 125.73 78.74) (width 1) (layer B.Cu) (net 3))
 (segment (start 166.175 117.87) (end 167.64 116.405) (width 1) (layer B.Cu) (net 3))
 (segment (start 163.195 117.87) (end 166.175 117.87) (width 1) (layer B.Cu) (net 3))
 (segment (start 167.64 116.405) (end 167.64 90.17) (width 1) (layer B.Cu) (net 3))
 (segment (start 166.37 88.9) (end 165.1 88.9) (width 1) (layer B.Cu) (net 3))
 (segment (start 167.64 90.17) (end 166.37 88.9) (width 1) (layer B.Cu) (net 3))
 (segment (start 80.520792 91.44) (end 79.248 91.44) (width 1) (layer B.Cu) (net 3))
 (segment (start 81.525 91.44) (end 80.520792 91.44) (width 1) (layer B.Cu) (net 3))
 (segment (start 91.12 81.845) (end 81.525 91.44) (width 1) (layer B.Cu) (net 3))
 (segment (start 91.12 79.945) (end 91.12 81.845) (width 1) (layer B.Cu) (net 3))
 (segment (start 140.97 116.84) (end 128.27 116.84) (width 1) (layer F.Cu) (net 8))
 (segment (start 128.27 116.84) (end 125.035 113.605) (width 1) (layer F.Cu) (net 8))
 (segment (start 144.145 114.935) (end 148.655 114.935) (width 0.5) (layer F.Cu) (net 8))
 (segment (start 140.97 116.84) (end 142.24 116.84) (width 0.5) (layer F.Cu) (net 8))
 (segment (start 142.24 116.84) (end 144.145 114.935) (width 0.5) (layer F.Cu) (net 8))
 (segment (start 148.655 114.935) (end 150.495 114.935) (width 0.5) (layer F.Cu) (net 8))
 (segment (start 151.05 114.38) (end 151.05 110.49) (width 0.5) (layer F.Cu) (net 8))
 (segment (start 150.495 114.935) (end 151.05 114.38) (width 0.5) (layer F.Cu) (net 8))
 (segment (start 135.255 101.68) (end 133.43 103.505) (width 0.5) (layer B.Cu) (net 8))
 (segment (start 135.255 100.33) (end 135.255 101.68) (width 0.5) (layer B.Cu) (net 8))
 (segment (start 133.43 103.505) (end 128.905 103.505) (width 0.5) (layer B.Cu) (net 8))
 (via (at 127 105.41) (size 0.8) (drill 0.4) (layers F.Cu B.Cu) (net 8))
 (segment (start 128.905 103.505) (end 127 105.41) (width 0.5) (layer B.Cu) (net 8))
 (segment (start 127 111.125) (end 124.46 113.665) (width 0.5) (layer F.Cu) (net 8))
 (segment (start 127 105.41) (end 127 111.125) (width 0.5) (layer F.Cu) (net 8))
 (segment (start 125.035 113.605) (end 124.46 113.665) (width 1) (layer F.Cu) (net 8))
 (segment (start 124.46 113.665) (end 122.867 113.605) (width 1) (layer F.Cu) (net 8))
 (segment (start 122.867 103.445) (end 125.79 103.445) (width 0.5) (layer B.Cu) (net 12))
 (segment (start 128.905 100.33) (end 132.715 100.33) (width 0.5) (layer B.Cu) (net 12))
 (segment (start 125.79 103.445) (end 128.905 100.33) (width 0.5) (layer B.Cu) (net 12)))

